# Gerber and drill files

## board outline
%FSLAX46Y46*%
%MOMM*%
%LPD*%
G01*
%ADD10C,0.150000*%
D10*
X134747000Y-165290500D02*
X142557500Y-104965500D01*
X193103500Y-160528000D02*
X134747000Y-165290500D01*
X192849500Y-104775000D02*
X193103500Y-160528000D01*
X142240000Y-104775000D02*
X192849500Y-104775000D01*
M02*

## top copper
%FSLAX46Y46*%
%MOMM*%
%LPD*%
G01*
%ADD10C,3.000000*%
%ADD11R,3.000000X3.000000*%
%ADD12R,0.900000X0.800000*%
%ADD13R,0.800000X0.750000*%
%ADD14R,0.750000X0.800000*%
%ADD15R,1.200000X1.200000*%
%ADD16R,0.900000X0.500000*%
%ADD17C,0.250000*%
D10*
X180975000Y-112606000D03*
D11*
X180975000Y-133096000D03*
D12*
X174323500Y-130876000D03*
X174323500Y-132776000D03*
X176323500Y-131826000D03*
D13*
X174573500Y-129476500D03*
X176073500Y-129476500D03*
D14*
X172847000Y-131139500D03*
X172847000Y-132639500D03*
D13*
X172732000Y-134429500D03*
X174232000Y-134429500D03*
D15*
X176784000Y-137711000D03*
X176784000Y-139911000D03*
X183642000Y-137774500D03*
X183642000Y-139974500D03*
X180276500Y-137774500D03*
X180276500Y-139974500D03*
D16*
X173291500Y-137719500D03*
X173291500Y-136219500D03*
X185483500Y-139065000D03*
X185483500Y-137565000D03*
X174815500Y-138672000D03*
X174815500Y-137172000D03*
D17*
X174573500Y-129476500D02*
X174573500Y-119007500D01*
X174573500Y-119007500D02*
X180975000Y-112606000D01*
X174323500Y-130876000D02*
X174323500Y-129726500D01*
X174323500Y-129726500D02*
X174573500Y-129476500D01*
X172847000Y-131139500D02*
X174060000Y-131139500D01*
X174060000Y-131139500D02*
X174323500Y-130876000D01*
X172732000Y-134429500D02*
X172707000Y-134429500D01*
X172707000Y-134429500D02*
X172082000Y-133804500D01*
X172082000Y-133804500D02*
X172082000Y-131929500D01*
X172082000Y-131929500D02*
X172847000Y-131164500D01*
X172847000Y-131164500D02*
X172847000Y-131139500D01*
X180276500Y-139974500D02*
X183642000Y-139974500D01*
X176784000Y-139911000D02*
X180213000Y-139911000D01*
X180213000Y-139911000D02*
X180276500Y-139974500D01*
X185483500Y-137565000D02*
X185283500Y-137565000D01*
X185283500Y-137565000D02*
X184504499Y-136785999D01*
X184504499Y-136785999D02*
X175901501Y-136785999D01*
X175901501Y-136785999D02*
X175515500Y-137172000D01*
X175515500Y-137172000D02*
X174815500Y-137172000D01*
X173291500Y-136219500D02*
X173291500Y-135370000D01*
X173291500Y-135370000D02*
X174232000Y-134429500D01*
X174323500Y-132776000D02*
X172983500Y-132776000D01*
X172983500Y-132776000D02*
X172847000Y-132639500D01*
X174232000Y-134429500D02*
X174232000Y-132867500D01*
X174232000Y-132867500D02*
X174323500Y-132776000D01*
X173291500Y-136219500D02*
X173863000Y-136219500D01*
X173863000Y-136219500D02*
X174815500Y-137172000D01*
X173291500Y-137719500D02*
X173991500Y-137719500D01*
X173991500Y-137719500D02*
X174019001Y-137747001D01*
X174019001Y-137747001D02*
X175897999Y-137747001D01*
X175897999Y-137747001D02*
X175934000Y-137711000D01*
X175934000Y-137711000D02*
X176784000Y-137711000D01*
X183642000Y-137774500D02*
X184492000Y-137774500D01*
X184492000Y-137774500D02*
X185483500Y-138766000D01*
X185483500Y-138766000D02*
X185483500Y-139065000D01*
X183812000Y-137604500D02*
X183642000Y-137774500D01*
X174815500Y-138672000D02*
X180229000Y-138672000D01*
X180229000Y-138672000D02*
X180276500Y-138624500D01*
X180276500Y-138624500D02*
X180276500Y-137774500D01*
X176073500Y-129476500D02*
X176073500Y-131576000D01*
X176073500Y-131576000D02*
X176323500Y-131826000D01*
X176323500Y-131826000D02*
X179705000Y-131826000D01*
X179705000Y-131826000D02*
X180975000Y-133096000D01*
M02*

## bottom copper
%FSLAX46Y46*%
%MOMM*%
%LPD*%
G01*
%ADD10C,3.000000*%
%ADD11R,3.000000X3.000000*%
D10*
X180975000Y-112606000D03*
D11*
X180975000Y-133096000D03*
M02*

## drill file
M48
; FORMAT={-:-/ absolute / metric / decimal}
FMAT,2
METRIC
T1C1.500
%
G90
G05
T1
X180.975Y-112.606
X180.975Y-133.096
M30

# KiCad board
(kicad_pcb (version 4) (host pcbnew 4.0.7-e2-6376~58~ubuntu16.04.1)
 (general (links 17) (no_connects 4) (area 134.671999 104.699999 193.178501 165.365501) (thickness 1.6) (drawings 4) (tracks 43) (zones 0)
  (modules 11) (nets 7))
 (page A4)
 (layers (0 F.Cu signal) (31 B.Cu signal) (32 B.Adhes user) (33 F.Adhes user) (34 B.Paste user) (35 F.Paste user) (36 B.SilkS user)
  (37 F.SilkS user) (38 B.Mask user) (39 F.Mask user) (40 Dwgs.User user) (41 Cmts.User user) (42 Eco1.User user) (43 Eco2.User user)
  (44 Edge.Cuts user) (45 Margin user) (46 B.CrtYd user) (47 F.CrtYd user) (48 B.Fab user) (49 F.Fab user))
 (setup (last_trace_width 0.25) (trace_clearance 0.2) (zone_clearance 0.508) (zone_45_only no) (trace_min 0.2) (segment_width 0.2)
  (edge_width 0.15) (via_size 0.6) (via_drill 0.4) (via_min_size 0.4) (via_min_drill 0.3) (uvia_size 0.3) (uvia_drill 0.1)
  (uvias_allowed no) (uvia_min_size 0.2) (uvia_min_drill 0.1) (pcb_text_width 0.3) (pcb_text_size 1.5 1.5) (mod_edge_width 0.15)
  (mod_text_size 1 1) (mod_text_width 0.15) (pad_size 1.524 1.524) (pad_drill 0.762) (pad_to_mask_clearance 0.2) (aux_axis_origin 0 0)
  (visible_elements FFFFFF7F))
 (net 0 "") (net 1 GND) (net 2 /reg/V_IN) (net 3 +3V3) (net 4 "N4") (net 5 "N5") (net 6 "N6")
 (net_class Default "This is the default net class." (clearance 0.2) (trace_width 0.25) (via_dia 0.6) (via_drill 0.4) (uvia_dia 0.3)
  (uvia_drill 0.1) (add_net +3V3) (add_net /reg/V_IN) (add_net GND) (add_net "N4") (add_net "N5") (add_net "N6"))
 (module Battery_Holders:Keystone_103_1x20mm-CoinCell (layer F.Cu) (at 180.975 133.096 90)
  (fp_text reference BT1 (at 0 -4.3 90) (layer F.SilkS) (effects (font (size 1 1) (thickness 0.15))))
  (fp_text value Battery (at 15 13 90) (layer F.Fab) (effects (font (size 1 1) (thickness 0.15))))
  (pad 2 thru_hole circle (at 20.49 0 90) (size 3 3) (drill 1.5) (layers *.Cu *.Mask) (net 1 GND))
  (pad 1 thru_hole rect (at 0 0 90) (size 3 3) (drill 1.5) (layers *.Cu *.Mask) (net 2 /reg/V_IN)))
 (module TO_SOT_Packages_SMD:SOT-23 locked (layer F.Cu) (at 175.3235 131.826)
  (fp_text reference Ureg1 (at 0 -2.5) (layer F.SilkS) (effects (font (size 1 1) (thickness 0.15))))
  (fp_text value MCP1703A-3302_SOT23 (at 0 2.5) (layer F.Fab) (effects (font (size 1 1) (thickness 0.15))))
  (pad 1 smd rect (at -1 -0.95) (size 0.9 0.8) (layers F.Cu F.Paste F.Mask) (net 1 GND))
  (pad 2 smd rect (at -1 0.95) (size 0.9 0.8) (layers F.Cu F.Paste F.Mask) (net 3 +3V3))
  (pad 3 smd rect (at 1 0) (size 0.9 0.8) (layers F.Cu F.Paste F.Mask) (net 2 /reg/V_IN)))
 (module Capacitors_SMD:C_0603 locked (layer F.Cu) (at 175.3235 129.4765 180)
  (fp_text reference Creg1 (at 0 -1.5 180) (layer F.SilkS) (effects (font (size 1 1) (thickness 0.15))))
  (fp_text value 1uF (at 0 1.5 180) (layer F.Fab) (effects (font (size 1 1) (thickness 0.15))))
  (pad 2 smd rect (at 0.75 0 180) (size 0.8 0.75) (layers F.Cu F.Paste F.Mask) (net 1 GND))
  (pad 1 smd rect (at -0.75 0 180) (size 0.8 0.75) (layers F.Cu F.Paste F.Mask) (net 2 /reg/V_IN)))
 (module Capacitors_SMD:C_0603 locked (layer F.Cu) (at 172.847 131.8895 90)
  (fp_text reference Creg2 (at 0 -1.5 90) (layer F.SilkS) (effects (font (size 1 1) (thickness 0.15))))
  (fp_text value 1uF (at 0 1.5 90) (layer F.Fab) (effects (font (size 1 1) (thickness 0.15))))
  (pad 2 smd rect (at 0.75 0 90) (size 0.8 0.75) (layers F.Cu F.Paste F.Mask) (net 1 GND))
  (pad 1 smd rect (at -0.75 0 90) (size 0.8 0.75) (layers F.Cu F.Paste F.Mask) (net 3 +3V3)))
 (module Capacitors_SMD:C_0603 (layer F.Cu) (at 173.482 134.4295 180)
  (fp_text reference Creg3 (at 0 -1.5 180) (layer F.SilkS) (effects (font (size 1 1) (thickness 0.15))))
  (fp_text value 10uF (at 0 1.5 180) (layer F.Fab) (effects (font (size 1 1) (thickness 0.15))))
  (pad 2 smd rect (at 0.75 0 180) (size 0.8 0.75) (layers F.Cu F.Paste F.Mask) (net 1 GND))
  (pad 1 smd rect (at -0.75 0 180) (size 0.8 0.75) (layers F.Cu F.Paste F.Mask) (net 3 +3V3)))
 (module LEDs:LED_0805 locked (layer F.Cu) (at 176.784 138.811 90)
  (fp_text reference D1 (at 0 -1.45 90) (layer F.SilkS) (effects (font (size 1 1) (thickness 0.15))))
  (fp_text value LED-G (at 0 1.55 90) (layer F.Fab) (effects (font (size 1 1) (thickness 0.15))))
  (pad 2 smd rect (at 1.1 0 270) (size 1.2 1.2) (layers F.Cu F.Paste F.Mask) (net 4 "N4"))
  (pad 1 smd rect (at -1.1 0 270) (size 1.2 1.2) (layers F.Cu F.Paste F.Mask) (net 1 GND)))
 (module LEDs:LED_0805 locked (layer F.Cu) (at 183.642 138.8745 90)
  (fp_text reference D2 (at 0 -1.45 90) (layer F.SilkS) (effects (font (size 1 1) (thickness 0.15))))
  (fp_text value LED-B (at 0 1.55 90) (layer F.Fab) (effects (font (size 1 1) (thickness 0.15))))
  (pad 2 smd rect (at 1.1 0 270) (size 1.2 1.2) (layers F.Cu F.Paste F.Mask) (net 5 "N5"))
  (pad 1 smd rect (at -1.1 0 270) (size 1.2 1.2) (layers F.Cu F.Paste F.Mask) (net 1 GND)))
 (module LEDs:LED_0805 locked (layer F.Cu) (at 180.2765 138.8745 90)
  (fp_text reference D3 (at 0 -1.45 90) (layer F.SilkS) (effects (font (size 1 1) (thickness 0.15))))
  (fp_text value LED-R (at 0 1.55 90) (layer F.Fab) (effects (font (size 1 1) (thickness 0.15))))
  (pad 2 smd rect (at 1.1 0 270) (size 1.2 1.2) (layers F.Cu F.Paste F.Mask) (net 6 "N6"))
  (pad 1 smd rect (at -1.1 0 270) (size 1.2 1.2) (layers F.Cu F.Paste F.Mask) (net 1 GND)))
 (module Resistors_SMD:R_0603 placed (layer F.Cu) (at 173.2915 136.9695 90)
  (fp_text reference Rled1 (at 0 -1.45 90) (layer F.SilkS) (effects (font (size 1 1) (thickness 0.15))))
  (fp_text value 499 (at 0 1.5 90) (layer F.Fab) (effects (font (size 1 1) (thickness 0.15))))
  (pad 1 smd rect (at -0.75 0 90) (size 0.5 0.9) (layers F.Cu F.Paste F.Mask) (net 4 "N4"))
  (pad 2 smd rect (at 0.75 0 90) (size 0.5 0.9) (layers F.Cu F.Paste F.Mask) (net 3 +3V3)))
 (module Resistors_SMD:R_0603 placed (layer F.Cu) (at 185.4835 138.315 90)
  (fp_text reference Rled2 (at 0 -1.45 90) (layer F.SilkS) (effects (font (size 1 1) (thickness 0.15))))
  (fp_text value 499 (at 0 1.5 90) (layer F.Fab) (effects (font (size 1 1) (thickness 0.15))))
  (pad 1 smd rect (at -0.75 0 90) (size 0.5 0.9) (layers F.Cu F.Paste F.Mask) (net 5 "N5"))
  (pad 2 smd rect (at 0.75 0 90) (size 0.5 0.9) (layers F.Cu F.Paste F.Mask) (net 3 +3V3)))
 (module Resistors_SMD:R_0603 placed (layer F.Cu) (at 174.8155 137.922 90)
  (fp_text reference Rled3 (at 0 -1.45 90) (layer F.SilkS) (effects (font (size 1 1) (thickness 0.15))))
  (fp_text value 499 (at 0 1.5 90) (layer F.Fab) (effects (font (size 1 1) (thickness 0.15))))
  (pad 1 smd rect (at -0.75 0 90) (size 0.5 0.9) (layers F.Cu F.Paste F.Mask) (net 6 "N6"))
  (pad 2 smd rect (at 0.75 0 90) (size 0.5 0.9) (layers F.Cu F.Paste F.Mask) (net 3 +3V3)))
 (gr_line (start 134.747 165.2905) (end 142.5575 104.9655) (layer Edge.Cuts) (width 0.15))
 (gr_line (start 193.1035 160.528) (end 134.747 165.2905) (layer Edge.Cuts) (width 0.15))
 (gr_line (start 192.8495 104.775) (end 193.1035 160.528) (layer Edge.Cuts) (width 0.15))
 (gr_line (start 142.24 104.775) (end 192.8495 104.775) (layer Edge.Cuts) (width 0.15))
 (segment (start 174.5735 129.4765) (end 174.5735 119.0075) (width 0.25) (layer F.Cu) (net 1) (status 10))
 (segment (start 174.5735 119.0075) (end 180.975 112.606) (width 0.25) (layer F.Cu) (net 1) (status 20))
 (segment (start 174.3235 130.876) (end 174.3235 129.7265) (width 0.25) (layer F.Cu) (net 1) (status 30))
 (segment (start 174.3235 129.7265) (end 174.5735 129.4765) (width 0.25) (layer F.Cu) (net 1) (status 30))
 (segment (start 172.847 131.1395) (end 174.06 131.1395) (width 0.25) (layer F.Cu) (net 1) (status 30))
 (segment (start 174.06 131.1395) (end 174.3235 130.876) (width 0.25) (layer F.Cu) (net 1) (status 30))
 (segment (start 172.732 134.4295) (end 172.707 134.4295) (width 0.25) (layer F.Cu) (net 1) (status 30))
 (segment (start 172.707 134.4295) (end 172.082 133.8045) (width 0.25) (layer F.Cu) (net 1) (status 10))
 (segment (start 172.082 133.8045) (end 172.082 131.9295) (width 0.25) (layer F.Cu) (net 1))
 (segment (start 172.082 131.9295) (end 172.847 131.1645) (width 0.25) (layer F.Cu) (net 1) (status 20))
 (segment (start 172.847 131.1645) (end 172.847 131.1395) (width 0.25) (layer F.Cu) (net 1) (status 30))
 (segment (start 180.2765 139.9745) (end 183.642 139.9745) (width 0.25) (layer F.Cu) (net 1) (status 30))
 (segment (start 176.784 139.911) (end 180.213 139.911) (width 0.25) (layer F.Cu) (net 1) (status 30))
 (segment (start 180.213 139.911) (end 180.2765 139.9745) (width 0.25) (layer F.Cu) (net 1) (status 30))
 (segment (start 185.4835 137.565) (end 185.2835 137.565) (width 0.25) (layer F.Cu) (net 3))
 (segment (start 185.2835 137.565) (end 184.504499 136.785999) (width 0.25) (layer F.Cu) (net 3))
 (segment (start 184.504499 136.785999) (end 175.901501 136.785999) (width 0.25) (layer F.Cu) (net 3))
 (segment (start 175.901501 136.785999) (end 175.5155 137.172) (width 0.25) (layer F.Cu) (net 3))
 (segment (start 175.5155 137.172) (end 174.8155 137.172) (width 0.25) (layer F.Cu) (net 3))
 (segment (start 173.2915 136.2195) (end 173.2915 135.37) (width 0.25) (layer F.Cu) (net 3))
 (segment (start 173.2915 135.37) (end 174.232 134.4295) (width 0.25) (layer F.Cu) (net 3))
 (segment (start 174.3235 132.776) (end 172.9835 132.776) (width 0.25) (layer F.Cu) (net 3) (status 30))
 (segment (start 172.9835 132.776) (end 172.847 132.6395) (width 0.25) (layer F.Cu) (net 3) (status 30))
 (segment (start 174.232 134.4295) (end 174.232 132.8675) (width 0.25) (layer F.Cu) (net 3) (status 30))
 (segment (start 174.232 132.8675) (end 174.3235 132.776) (width 0.25) (layer F.Cu) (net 3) (status 30))
 (segment (start 173.2915 136.2195) (end 173.863 136.2195) (width 0.25) (layer F.Cu) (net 3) (status 10))
 (segment (start 173.863 136.2195) (end 174.8155 137.172) (width 0.25) (layer F.Cu) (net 3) (status 20))
 (segment (start 173.2915 137.7195) (end 173.9915 137.7195) (width 0.25) (layer F.Cu) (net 4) (status 10))
 (segment (start 173.9915 137.7195) (end 174.019001 137.747001) (width 0.25) (layer F.Cu) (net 4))
 (segment (start 174.019001 137.747001) (end 175.897999 137.747001) (width 0.25) (layer F.Cu) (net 4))
 (segment (start 175.897999 137.747001) (end 175.934 137.711) (width 0.25) (layer F.Cu) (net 4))
 (segment (start 175.934 137.711) (end 176.784 137.711) (width 0.25) (layer F.Cu) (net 4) (status 20))
 (segment (start 183.642 137.7745) (end 184.492 137.7745) (width 0.25) (layer F.Cu) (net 5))
 (segment (start 184.492 137.7745) (end 185.4835 138.766) (width 0.25) (layer F.Cu) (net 5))
 (segment (start 185.4835 138.766) (end 185.4835 139.065) (width 0.25) (layer F.Cu) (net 5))
 (segment (start 183.812 137.6045) (end 183.642 137.7745) (width 0.25) (layer F.Cu) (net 5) (status 30))
 (segment (start 174.8155 138.672) (end 180.229 138.672) (width 0.25) (layer F.Cu) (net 6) (status 10))
 (segment (start 180.229 138.672) (end 180.2765 138.6245) (width 0.25) (layer F.Cu) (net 6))
 (segment (start 180.2765 138.6245) (end 180.2765 137.7745) (width 0.25) (layer F.Cu) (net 6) (status 20))
 (segment (start 176.0735 129.4765) (end 176.0735 131.576) (width 0.25) (layer F.Cu) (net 2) (status 30))
 (segment (start 176.0735 131.576) (end 176.3235 131.826) (width 0.25) (layer F.Cu) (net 2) (status 30))
 (segment (start 176.3235 131.826) (end 179.705 131.826) (width 0.25) (layer F.Cu) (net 2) (status 30))
 (segment (start 179.705 131.826) (end 180.975 133.096) (width 0.25) (layer F.Cu) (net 2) (status 30)))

